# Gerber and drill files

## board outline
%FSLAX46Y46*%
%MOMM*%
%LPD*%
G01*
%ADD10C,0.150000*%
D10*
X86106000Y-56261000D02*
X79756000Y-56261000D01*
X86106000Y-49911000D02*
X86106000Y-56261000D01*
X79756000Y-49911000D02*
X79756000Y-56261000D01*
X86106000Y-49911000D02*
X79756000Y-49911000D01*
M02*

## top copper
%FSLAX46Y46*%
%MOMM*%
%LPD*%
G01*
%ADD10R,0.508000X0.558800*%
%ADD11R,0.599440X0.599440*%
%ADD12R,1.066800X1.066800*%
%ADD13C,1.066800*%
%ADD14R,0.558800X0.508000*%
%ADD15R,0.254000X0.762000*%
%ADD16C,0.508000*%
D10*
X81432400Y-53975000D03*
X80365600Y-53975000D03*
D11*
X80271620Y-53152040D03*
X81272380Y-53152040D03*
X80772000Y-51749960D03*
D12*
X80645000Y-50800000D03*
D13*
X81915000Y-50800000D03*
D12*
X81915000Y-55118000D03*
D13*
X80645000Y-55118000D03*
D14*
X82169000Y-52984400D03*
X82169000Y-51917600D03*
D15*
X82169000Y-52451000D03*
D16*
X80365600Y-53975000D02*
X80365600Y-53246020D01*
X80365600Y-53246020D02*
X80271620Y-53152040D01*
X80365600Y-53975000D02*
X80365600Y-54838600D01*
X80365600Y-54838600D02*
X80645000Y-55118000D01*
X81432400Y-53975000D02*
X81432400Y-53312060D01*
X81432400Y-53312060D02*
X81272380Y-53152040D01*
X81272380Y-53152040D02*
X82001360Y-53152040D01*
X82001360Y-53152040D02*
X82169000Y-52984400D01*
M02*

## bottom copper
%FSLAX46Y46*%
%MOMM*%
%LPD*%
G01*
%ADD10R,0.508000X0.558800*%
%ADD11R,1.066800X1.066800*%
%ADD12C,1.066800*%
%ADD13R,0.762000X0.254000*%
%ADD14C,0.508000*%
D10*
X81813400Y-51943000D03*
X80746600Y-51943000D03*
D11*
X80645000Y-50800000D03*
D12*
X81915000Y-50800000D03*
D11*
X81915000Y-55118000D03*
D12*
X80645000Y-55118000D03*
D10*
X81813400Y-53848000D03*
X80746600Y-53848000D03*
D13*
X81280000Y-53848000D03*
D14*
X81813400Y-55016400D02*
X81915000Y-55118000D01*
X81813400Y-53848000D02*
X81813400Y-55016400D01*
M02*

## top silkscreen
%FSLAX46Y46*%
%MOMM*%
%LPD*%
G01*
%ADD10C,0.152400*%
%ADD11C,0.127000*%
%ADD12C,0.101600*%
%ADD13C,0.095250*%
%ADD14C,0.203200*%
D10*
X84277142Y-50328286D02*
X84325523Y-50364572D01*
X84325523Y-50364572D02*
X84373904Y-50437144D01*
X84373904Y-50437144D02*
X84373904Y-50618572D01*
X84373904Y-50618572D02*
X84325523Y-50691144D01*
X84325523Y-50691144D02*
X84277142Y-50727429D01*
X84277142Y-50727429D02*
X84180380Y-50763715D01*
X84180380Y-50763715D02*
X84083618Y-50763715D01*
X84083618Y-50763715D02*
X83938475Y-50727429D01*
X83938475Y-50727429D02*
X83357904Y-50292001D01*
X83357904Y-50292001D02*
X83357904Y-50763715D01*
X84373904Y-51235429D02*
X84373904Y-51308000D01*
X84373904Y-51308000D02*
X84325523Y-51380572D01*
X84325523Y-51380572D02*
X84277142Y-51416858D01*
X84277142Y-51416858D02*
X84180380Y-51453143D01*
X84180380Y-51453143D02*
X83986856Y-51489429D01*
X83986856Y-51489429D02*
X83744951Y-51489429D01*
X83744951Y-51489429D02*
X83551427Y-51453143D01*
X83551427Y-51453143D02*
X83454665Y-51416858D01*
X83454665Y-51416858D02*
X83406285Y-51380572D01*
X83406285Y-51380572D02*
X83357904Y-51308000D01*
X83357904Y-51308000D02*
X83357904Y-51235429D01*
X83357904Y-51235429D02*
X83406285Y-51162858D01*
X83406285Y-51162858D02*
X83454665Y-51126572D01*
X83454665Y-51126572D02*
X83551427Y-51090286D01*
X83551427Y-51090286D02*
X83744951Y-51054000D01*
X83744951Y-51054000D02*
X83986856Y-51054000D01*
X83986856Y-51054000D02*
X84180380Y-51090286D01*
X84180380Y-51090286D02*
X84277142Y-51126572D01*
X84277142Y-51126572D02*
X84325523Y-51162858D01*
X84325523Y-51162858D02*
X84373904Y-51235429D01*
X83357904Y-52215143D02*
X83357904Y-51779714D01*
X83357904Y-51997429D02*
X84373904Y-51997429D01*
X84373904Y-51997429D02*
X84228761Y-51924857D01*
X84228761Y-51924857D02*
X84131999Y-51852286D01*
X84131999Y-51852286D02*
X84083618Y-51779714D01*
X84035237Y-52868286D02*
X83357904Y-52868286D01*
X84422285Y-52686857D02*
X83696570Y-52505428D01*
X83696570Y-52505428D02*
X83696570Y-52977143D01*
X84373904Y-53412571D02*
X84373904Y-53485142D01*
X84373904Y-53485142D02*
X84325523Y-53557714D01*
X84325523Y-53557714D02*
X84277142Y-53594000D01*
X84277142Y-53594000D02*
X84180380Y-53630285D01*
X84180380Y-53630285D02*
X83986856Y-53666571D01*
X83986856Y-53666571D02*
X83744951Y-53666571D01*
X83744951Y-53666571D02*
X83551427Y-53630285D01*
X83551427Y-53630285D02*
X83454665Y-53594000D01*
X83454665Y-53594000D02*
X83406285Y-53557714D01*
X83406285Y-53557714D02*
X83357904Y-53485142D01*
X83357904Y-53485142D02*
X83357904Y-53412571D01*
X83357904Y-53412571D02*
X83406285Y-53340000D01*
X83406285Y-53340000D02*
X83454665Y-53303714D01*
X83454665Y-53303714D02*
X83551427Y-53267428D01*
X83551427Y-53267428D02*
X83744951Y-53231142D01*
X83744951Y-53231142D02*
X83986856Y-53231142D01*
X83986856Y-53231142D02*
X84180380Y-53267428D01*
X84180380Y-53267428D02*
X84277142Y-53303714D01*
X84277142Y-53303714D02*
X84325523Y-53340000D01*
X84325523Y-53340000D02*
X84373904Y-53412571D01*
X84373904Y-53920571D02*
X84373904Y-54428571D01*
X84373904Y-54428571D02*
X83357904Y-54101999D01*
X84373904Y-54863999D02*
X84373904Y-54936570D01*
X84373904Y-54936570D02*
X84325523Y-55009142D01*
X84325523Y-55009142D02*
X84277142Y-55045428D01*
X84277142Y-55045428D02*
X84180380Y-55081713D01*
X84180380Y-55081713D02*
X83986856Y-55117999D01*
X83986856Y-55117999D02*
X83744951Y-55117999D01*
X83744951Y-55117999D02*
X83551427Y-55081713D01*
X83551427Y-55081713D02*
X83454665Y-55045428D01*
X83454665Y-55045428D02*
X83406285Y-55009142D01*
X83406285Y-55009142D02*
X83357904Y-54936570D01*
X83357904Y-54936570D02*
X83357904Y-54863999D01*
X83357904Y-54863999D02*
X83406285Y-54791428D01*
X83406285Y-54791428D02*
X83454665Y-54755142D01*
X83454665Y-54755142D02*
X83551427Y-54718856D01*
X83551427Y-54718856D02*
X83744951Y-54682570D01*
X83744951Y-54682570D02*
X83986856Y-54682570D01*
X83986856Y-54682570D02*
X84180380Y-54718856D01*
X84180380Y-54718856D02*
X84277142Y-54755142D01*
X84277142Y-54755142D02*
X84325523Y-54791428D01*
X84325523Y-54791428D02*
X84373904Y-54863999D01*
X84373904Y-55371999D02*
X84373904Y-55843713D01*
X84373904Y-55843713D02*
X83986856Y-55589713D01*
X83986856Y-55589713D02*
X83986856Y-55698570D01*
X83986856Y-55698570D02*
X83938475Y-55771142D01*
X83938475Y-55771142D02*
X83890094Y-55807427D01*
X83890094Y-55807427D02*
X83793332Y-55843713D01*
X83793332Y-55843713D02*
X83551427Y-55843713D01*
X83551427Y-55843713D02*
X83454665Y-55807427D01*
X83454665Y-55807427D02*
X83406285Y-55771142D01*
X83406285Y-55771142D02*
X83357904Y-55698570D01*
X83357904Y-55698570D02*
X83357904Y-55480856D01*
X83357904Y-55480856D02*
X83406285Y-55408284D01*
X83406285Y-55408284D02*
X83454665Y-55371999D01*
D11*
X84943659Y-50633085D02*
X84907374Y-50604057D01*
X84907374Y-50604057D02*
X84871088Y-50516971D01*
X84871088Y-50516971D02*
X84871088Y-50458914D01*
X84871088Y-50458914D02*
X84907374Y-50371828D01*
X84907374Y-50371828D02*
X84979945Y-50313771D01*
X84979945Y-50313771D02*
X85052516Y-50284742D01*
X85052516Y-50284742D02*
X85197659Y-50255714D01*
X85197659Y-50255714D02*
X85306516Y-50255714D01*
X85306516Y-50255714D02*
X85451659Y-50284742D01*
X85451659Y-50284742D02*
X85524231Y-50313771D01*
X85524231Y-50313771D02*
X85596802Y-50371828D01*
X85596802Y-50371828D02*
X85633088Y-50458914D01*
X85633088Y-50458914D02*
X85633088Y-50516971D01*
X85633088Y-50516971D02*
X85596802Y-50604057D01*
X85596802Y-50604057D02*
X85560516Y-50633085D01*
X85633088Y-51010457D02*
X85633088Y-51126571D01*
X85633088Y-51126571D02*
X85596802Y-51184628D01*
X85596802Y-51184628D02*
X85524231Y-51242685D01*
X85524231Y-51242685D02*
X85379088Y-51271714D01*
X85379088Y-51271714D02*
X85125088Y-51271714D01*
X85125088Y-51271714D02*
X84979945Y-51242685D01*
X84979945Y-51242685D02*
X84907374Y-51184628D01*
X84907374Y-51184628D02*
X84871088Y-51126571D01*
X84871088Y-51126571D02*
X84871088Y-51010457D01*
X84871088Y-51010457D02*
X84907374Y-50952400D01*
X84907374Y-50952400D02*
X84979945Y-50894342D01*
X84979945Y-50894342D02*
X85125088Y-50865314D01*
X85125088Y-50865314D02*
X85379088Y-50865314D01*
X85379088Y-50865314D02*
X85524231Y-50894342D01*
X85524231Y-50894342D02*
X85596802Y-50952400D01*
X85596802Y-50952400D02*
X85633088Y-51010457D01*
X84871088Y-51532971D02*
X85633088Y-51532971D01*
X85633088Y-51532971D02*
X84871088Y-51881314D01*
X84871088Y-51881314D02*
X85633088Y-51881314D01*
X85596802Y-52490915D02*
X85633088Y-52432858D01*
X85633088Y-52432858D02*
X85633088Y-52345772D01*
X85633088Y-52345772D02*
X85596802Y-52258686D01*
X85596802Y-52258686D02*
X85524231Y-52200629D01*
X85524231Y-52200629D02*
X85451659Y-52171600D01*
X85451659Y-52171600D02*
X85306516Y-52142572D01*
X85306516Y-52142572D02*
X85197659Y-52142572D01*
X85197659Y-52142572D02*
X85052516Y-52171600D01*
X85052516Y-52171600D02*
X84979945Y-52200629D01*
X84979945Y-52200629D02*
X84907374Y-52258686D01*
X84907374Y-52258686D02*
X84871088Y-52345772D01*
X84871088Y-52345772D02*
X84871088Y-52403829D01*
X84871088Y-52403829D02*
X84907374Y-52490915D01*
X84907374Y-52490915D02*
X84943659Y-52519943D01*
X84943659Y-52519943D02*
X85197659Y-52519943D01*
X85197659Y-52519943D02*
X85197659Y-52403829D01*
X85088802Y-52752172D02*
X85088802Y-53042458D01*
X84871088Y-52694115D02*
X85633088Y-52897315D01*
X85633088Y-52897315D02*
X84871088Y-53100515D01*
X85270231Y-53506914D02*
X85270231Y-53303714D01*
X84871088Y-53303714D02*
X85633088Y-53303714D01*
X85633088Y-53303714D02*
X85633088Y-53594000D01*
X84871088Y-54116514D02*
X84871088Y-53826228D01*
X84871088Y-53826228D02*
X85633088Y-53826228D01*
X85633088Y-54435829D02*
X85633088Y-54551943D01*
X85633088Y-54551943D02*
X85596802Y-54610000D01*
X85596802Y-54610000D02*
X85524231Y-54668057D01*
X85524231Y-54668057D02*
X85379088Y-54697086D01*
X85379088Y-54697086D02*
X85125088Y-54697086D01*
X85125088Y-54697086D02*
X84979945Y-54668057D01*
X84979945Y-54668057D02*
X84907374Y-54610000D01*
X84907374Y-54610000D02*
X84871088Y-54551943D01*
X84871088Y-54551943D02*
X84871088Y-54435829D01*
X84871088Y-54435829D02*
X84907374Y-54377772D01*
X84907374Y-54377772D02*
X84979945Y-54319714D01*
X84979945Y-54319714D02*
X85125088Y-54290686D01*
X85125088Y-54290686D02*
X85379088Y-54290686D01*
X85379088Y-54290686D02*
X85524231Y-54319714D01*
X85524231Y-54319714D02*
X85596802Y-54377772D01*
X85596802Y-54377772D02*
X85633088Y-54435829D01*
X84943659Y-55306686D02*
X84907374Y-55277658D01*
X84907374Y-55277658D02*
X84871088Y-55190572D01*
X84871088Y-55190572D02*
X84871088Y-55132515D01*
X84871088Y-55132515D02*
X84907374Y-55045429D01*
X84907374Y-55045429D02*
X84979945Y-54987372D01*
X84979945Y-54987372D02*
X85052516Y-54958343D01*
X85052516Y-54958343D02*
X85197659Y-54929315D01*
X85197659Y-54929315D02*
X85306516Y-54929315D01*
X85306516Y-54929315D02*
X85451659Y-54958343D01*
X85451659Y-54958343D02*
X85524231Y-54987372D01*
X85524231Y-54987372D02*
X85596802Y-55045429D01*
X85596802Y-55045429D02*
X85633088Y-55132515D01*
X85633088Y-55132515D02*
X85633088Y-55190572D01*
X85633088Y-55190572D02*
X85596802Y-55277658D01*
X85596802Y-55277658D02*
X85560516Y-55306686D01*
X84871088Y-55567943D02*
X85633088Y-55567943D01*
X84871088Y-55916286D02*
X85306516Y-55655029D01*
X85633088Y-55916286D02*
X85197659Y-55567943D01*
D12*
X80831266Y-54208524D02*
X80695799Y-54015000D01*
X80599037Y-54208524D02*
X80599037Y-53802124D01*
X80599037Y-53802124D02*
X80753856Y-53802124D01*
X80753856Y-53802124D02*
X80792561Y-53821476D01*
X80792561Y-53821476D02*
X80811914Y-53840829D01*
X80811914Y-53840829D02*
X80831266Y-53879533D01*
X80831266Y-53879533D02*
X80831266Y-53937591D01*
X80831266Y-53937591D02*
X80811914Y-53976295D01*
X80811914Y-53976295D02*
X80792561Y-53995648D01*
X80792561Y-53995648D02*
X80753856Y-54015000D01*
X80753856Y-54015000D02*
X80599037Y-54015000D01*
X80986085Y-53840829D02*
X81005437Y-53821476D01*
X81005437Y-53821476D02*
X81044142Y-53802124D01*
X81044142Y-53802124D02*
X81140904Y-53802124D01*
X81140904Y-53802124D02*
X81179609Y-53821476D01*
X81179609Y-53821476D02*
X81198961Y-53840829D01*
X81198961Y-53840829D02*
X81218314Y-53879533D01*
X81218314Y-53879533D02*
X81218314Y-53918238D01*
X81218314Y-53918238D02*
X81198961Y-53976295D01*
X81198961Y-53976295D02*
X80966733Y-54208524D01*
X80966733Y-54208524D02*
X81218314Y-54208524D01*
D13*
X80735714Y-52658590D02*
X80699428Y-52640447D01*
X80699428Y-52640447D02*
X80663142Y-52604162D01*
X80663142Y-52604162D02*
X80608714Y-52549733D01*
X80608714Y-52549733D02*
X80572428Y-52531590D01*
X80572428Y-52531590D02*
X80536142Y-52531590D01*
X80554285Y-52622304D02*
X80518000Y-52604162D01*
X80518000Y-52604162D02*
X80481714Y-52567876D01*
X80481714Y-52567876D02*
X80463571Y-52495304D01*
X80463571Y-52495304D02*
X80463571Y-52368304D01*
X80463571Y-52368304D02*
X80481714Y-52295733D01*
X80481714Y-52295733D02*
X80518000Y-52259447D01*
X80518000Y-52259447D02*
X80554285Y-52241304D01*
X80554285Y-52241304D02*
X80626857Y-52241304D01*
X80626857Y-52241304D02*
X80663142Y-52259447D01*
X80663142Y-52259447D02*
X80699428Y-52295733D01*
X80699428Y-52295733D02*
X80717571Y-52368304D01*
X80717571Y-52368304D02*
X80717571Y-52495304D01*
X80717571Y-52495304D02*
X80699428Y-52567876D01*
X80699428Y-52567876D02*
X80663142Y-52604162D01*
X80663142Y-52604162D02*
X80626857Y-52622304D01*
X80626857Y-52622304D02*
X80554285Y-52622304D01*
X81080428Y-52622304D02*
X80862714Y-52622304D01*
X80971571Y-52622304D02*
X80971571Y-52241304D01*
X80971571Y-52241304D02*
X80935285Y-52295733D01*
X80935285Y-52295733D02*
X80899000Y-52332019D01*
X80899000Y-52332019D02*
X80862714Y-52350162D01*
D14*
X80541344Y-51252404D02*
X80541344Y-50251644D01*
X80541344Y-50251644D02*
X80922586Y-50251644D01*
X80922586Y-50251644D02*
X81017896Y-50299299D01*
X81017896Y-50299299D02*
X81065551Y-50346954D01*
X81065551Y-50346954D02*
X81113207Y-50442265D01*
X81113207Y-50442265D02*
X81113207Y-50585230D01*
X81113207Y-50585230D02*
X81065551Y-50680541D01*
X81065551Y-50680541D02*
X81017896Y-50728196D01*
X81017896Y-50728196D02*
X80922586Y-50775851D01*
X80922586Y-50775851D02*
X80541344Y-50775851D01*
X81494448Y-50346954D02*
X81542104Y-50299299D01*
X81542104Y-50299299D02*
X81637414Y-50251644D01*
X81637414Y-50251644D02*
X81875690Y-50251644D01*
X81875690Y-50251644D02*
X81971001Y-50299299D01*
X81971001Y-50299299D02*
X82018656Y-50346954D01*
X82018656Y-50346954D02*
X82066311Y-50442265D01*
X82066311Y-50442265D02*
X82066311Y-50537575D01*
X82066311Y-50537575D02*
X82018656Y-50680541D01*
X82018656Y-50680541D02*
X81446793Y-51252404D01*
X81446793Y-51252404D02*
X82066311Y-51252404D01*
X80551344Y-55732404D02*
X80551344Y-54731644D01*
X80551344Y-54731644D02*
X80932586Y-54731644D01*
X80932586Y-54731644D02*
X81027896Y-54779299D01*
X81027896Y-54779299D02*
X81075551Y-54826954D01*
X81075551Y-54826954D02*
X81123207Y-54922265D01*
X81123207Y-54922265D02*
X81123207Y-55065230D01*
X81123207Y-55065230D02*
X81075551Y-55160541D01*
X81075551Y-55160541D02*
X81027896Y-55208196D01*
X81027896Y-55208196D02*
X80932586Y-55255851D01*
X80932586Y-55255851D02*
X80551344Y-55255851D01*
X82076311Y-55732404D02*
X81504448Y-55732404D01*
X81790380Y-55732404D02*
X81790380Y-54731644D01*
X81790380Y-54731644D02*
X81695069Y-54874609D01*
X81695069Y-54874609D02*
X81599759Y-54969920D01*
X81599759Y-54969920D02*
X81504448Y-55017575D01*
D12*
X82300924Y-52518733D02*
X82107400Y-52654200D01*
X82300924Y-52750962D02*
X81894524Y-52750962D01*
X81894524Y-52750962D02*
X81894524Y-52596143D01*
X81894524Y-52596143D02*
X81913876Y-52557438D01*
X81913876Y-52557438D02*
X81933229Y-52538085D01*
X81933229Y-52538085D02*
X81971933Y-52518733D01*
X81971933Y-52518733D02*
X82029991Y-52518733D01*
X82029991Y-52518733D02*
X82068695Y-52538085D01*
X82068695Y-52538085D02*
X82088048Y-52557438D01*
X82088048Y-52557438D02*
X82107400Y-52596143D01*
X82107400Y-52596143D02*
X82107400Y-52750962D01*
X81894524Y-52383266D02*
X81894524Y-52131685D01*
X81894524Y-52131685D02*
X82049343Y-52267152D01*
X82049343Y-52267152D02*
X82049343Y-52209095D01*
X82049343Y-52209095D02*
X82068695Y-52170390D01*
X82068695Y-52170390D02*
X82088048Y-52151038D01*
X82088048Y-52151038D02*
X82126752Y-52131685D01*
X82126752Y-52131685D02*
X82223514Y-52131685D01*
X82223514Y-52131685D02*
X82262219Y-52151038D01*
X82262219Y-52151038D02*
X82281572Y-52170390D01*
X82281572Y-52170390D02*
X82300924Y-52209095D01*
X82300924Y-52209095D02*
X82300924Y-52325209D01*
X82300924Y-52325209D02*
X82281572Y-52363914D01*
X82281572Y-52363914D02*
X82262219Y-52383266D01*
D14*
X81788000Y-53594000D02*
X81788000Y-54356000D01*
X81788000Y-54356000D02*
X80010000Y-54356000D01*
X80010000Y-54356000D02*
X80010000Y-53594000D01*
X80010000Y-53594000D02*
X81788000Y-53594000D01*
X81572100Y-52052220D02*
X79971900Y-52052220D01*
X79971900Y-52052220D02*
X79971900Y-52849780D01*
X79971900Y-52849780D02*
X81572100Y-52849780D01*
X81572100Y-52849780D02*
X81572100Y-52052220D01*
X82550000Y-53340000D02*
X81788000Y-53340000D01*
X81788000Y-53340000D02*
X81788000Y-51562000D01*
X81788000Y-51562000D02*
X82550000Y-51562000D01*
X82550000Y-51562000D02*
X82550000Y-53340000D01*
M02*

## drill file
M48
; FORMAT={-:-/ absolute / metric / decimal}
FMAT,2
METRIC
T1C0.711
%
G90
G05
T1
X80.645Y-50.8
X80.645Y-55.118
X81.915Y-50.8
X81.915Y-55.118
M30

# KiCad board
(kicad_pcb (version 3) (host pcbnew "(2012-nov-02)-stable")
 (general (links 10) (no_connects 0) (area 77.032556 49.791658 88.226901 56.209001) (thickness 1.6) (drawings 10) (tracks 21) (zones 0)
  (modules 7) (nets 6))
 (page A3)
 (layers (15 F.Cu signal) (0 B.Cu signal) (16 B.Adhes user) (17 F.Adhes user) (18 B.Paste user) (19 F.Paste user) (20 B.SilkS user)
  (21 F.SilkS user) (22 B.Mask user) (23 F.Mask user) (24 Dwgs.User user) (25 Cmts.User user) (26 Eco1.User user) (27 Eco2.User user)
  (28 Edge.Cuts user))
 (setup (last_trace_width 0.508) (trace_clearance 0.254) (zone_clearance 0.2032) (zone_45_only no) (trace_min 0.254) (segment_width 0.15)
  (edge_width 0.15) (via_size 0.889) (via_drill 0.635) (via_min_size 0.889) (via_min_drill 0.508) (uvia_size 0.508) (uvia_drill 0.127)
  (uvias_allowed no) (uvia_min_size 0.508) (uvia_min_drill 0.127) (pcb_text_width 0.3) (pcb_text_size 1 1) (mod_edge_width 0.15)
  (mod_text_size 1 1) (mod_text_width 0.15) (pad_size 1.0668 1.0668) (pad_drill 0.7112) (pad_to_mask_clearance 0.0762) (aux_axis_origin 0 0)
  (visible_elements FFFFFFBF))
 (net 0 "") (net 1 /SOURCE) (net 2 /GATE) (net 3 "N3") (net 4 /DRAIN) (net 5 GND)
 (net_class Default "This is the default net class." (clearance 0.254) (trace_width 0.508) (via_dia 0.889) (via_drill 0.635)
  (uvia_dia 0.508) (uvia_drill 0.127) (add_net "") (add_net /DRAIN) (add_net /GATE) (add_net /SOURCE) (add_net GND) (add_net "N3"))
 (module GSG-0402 (layer F.Cu) (at 80.899 53.975) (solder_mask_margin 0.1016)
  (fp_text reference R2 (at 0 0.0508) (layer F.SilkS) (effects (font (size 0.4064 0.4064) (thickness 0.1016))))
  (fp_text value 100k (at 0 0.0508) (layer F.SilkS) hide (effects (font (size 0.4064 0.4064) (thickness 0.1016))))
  (fp_line (start 0.889 -0.381) (end 0.889 0.381) (layer F.SilkS) (width 0.2032))
  (fp_line (start 0.889 0.381) (end -0.889 0.381) (layer F.SilkS) (width 0.2032))
  (fp_line (start -0.889 0.381) (end -0.889 -0.381) (layer F.SilkS) (width 0.2032))
  (fp_line (start -0.889 -0.381) (end 0.889 -0.381) (layer F.SilkS) (width 0.2032))
  (pad 2 smd rect (at 0.5334 0) (size 0.508 0.5588) (layers F.Cu F.Paste F.Mask) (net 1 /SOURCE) (solder_mask_margin 0.1016))
  (pad 1 smd rect (at -0.5334 0) (size 0.508 0.5588) (layers F.Cu F.Paste F.Mask) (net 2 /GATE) (die_length -2147.483648)
   (solder_mask_margin 0.1016)))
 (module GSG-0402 (layer B.Cu) (at 81.28 51.943) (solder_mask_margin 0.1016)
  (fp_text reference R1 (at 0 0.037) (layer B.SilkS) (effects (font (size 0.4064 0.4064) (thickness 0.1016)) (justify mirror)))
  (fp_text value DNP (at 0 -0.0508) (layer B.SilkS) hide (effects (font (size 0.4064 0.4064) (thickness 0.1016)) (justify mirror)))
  (pad 2 smd rect (at 0.5334 0) (size 0.508 0.5588) (layers B.Cu B.Paste B.Mask) (solder_mask_margin 0.1016))
  (pad 1 smd rect (at -0.5334 0) (size 0.508 0.5588) (layers B.Cu B.Paste B.Mask) (die_length -2147.483648) (solder_mask_margin 0.1016)))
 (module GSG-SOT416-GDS (layer F.Cu) (at 80.772 52.451)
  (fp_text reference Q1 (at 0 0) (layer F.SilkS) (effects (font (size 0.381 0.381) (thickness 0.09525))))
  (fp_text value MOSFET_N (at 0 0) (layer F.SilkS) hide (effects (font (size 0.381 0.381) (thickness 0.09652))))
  (fp_line (start 0.8001 -0.39878) (end -0.8001 -0.39878) (layer F.SilkS) (width 0.2032))
  (fp_line (start -0.8001 -0.39878) (end -0.8001 0.39878) (layer F.SilkS) (width 0.2032))
  (fp_line (start -0.8001 0.39878) (end 0.8001 0.39878) (layer F.SilkS) (width 0.2032))
  (fp_line (start 0.8001 0.39878) (end 0.8001 -0.39878) (layer F.SilkS) (width 0.2032))
  (pad G smd rect (at -0.50038 0.70104) (size 0.59944 0.59944) (layers F.Cu F.Paste F.Mask) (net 2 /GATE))
  (pad S smd rect (at 0.50038 0.70104) (size 0.59944 0.59944) (layers F.Cu F.Paste F.Mask) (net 1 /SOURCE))
  (pad D smd rect (at 0 -0.70104) (size 0.59944 0.59944) (layers F.Cu F.Paste F.Mask)))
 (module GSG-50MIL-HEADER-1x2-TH (layer F.Cu) (at 81.28 50.8)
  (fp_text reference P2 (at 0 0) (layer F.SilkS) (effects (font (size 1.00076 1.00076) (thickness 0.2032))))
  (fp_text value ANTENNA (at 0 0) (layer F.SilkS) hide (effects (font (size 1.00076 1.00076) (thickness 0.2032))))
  (pad 1 thru_hole rect (at -0.635 0) (size 1.0668 1.0668) (drill 0.7112) (layers *.Cu *.Mask))
  (pad 2 thru_hole circle (at 0.635 0) (size 1.0668 1.0668) (drill 0.7112) (layers *.Cu *.Mask)))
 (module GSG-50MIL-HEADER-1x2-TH (layer F.Cu) (at 81.28 55.118 180)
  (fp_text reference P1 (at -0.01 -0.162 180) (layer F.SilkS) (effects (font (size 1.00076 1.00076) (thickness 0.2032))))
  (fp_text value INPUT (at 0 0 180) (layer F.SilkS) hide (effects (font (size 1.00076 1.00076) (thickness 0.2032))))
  (pad 1 thru_hole rect (at -0.635 0 180) (size 1.0668 1.0668) (drill 0.7112) (layers *.Cu *.Mask) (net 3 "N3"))
  (pad 2 thru_hole circle (at 0.635 0 180) (size 1.0668 1.0668) (drill 0.7112) (layers *.Cu *.Mask) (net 2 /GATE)))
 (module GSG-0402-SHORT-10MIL (layer B.Cu) (at 81.28 53.848) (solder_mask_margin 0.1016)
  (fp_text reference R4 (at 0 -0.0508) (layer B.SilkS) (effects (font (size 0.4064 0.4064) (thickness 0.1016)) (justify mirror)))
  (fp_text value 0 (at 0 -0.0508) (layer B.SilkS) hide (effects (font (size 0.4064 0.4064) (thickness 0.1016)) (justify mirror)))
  (pad 2 smd rect (at 0.5334 0) (size 0.508 0.5588) (layers B.Cu B.Mask) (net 3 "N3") (solder_mask_margin 0.1016))
  (pad 1 smd rect (at -0.5334 0) (size 0.508 0.5588) (layers B.Cu B.Mask) (die_length -2147.483648) (solder_mask_margin 0.1016))
  (pad "" smd rect (at 0 0) (size 0.762 0.254) (layers B.Cu B.Mask)))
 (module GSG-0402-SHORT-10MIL (layer F.Cu) (at 82.169 52.451 270) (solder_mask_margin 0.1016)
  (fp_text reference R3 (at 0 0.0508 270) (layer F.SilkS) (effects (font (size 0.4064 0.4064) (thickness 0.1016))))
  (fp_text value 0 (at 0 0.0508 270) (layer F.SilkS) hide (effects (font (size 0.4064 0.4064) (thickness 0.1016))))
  (fp_line (start 0.889 -0.381) (end 0.889 0.381) (layer F.SilkS) (width 0.2032))
  (fp_line (start 0.889 0.381) (end -0.889 0.381) (layer F.SilkS) (width 0.2032))
  (fp_line (start -0.889 0.381) (end -0.889 -0.381) (layer F.SilkS) (width 0.2032))
  (fp_line (start -0.889 -0.381) (end 0.889 -0.381) (layer F.SilkS) (width 0.2032))
  (pad 2 smd rect (at 0.5334 0 270) (size 0.508 0.5588) (layers F.Cu F.Mask) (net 1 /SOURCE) (solder_mask_margin 0.1016))
  (pad 1 smd rect (at -0.5334 0 270) (size 0.508 0.5588) (layers F.Cu F.Mask) (die_length -2147.483648) (solder_mask_margin 0.1016))
  (pad "" smd rect (at 0 0 270) (size 0.762 0.254) (layers F.Cu F.Mask)))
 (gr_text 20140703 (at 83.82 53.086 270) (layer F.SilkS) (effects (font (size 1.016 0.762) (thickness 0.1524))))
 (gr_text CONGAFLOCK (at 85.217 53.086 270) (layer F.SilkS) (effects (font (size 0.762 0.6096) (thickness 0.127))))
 (gr_line (start 86.106 56.261) (end 79.756 56.261) (angle 90) (layer Edge.Cuts) (width 0.15))
 (gr_line (start 86.106 49.911) (end 86.106 56.261) (angle 90) (layer Edge.Cuts) (width 0.15))
 (gr_line (start 79.756 49.911) (end 79.756 56.261) (angle 90) (layer Edge.Cuts) (width 0.15))
 (gr_line (start 86.106 49.911) (end 79.756 49.911) (angle 90) (layer Edge.Cuts) (width 0.15))
 (segment (start 80.3656 53.975) (end 80.3656 53.24602) (width 0.508) (layer F.Cu) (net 2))
 (segment (start 80.3656 53.24602) (end 80.27162 53.15204) (width 0.508) (layer F.Cu) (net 2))
 (segment (start 80.3656 53.975) (end 80.3656 54.8386) (width 0.508) (layer F.Cu) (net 2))
 (segment (start 80.3656 54.8386) (end 80.645 55.118) (width 0.508) (layer F.Cu) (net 2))
 (segment (start 81.4324 53.975) (end 81.4324 53.31206) (width 0.508) (layer F.Cu) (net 1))
 (segment (start 81.4324 53.31206) (end 81.27238 53.15204) (width 0.508) (layer F.Cu) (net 1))
 (segment (start 81.27238 53.15204) (end 82.00136 53.15204) (width 0.508) (layer F.Cu) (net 1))
 (segment (start 82.00136 53.15204) (end 82.169 52.9844) (width 0.508) (layer F.Cu) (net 1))
 (segment (start 81.8134 55.0164) (end 81.915 55.118) (width 0.508) (layer B.Cu) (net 3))
 (segment (start 81.8134 53.848) (end 81.8134 55.0164) (width 0.508) (layer B.Cu) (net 3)))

